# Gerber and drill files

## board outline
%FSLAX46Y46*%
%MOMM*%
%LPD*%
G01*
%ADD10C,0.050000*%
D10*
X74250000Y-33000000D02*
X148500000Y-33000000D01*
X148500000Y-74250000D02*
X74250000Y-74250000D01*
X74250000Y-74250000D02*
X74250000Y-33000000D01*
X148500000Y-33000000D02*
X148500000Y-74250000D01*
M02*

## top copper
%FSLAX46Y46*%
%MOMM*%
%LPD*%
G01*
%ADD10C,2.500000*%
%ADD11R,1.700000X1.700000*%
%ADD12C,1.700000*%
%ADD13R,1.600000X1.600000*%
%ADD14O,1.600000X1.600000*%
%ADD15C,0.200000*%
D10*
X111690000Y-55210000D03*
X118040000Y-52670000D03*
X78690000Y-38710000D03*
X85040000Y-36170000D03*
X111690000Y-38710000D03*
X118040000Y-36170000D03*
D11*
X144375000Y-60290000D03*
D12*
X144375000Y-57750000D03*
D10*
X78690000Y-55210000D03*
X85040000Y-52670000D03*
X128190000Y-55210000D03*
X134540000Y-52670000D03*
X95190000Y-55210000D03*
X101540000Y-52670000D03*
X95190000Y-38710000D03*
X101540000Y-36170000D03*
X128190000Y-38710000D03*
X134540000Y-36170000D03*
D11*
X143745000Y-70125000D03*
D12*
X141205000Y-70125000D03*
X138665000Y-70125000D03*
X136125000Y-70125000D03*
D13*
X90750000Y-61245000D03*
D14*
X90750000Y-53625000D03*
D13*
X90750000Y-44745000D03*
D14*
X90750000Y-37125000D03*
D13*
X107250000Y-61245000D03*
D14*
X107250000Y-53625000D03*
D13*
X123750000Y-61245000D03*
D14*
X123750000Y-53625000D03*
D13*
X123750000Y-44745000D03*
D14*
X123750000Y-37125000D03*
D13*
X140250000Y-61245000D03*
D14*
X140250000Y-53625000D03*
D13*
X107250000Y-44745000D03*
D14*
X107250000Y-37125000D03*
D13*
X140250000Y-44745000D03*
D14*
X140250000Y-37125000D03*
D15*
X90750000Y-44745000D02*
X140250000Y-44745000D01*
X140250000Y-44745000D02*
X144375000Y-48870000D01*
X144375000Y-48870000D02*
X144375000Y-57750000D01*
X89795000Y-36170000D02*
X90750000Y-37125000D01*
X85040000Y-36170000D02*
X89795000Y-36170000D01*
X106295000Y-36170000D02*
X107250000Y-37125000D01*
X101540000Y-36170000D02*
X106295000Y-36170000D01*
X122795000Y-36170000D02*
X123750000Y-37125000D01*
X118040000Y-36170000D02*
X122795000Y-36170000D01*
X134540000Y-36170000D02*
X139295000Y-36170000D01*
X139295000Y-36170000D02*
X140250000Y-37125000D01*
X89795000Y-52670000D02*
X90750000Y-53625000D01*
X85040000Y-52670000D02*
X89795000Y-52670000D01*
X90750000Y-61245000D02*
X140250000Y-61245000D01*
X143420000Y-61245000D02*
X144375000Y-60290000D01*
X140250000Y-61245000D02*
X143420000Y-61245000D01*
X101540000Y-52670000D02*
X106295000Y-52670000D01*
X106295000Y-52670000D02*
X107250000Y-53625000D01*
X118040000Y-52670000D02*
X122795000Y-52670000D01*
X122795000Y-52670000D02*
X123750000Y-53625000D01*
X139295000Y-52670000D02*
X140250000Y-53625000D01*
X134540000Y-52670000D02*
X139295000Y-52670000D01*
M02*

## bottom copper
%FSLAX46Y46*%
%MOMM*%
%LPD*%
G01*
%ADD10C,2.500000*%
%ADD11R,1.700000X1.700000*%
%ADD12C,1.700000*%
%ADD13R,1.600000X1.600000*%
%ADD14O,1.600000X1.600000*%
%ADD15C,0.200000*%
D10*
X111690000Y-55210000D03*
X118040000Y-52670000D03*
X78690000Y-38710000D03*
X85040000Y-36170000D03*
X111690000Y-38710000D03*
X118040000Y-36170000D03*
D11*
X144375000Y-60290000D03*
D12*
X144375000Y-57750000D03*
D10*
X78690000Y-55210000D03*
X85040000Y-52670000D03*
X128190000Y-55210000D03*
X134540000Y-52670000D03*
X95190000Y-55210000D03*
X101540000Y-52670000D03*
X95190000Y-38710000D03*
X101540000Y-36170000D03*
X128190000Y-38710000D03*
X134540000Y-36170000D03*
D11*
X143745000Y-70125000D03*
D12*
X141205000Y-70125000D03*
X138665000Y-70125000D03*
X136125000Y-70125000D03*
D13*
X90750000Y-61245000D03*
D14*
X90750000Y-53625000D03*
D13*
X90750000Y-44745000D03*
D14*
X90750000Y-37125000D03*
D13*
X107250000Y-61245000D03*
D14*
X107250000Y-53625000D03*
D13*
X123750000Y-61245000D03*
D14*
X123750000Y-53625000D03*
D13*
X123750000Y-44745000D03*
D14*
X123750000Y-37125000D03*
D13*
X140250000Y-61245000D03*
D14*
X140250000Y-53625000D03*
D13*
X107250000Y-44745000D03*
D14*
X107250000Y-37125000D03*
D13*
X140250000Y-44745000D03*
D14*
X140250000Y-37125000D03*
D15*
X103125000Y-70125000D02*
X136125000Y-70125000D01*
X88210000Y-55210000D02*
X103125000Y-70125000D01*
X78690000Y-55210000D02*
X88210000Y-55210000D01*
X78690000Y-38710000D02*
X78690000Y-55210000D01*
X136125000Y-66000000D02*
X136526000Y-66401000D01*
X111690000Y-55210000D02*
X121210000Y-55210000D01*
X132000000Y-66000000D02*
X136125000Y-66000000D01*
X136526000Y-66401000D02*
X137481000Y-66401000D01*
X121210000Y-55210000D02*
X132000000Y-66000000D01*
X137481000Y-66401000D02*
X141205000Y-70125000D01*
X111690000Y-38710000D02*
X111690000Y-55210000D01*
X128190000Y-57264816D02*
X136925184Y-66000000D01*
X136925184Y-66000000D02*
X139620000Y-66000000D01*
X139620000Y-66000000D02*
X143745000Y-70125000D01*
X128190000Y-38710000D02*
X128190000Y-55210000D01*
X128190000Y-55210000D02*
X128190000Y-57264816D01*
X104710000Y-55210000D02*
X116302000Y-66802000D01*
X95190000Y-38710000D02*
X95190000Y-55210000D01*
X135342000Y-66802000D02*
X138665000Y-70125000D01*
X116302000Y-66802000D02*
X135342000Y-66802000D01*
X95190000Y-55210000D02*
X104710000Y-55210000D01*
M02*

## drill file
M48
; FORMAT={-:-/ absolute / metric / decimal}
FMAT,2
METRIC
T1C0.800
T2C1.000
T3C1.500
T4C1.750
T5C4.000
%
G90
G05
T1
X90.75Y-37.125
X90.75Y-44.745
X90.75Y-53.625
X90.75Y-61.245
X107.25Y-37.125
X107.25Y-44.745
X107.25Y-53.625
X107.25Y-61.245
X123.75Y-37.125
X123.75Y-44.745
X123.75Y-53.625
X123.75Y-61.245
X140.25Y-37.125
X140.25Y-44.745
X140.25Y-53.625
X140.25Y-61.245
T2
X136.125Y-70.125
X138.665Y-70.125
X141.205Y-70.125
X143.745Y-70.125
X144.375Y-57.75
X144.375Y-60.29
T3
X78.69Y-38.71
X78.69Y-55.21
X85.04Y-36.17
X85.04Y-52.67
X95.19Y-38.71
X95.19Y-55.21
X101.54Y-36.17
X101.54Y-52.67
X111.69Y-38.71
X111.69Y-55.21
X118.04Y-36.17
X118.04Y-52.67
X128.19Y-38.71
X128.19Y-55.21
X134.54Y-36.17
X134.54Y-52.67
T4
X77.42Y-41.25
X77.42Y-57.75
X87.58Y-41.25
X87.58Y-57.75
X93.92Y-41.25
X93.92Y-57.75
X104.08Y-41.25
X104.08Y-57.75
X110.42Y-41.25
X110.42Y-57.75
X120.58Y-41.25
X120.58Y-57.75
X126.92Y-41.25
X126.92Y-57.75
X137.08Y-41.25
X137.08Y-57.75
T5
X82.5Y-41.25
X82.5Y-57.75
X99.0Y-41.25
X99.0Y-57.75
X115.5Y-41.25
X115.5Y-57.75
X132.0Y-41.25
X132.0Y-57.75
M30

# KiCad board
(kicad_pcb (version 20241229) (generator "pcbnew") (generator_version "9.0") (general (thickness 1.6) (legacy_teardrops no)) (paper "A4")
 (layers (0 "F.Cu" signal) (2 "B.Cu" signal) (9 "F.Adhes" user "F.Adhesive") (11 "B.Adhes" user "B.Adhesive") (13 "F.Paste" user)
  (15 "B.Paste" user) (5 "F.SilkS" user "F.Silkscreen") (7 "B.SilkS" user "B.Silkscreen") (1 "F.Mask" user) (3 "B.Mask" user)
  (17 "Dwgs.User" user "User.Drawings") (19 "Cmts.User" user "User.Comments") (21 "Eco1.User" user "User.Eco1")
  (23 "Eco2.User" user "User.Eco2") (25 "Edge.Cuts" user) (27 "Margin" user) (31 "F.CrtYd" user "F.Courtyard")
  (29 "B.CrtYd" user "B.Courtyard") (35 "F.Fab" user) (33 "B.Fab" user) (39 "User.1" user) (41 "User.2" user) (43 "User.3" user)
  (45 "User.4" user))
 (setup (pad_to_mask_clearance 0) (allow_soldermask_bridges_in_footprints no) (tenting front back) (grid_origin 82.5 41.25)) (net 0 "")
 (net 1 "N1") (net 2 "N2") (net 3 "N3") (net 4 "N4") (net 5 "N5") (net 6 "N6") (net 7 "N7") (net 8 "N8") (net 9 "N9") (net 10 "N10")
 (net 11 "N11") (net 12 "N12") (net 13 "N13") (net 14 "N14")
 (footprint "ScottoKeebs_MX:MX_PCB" (layer "F.Cu") (at 115.5 57.75)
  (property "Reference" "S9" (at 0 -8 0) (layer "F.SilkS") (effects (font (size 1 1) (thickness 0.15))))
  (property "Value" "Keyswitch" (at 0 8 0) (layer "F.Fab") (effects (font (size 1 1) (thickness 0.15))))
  (pad "" np_thru_hole circle (at -5.08 0) (size 1.75 1.75) (drill 1.75) (layers "*.Cu" "*.Mask"))
  (pad "" np_thru_hole circle (at 0 0) (size 4 4) (drill 4) (layers "*.Cu" "*.Mask"))
  (pad "" np_thru_hole circle (at 5.08 0) (size 1.75 1.75) (drill 1.75) (layers "*.Cu" "*.Mask"))
  (pad "1" thru_hole circle (at -3.81 -2.54) (size 2.5 2.5) (drill 1.5) (layers "*.Cu" "*.Mask") (remove_unused_layers no) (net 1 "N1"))
  (pad "2" thru_hole circle (at 2.54 -5.08) (size 2.5 2.5) (drill 1.5) (layers "*.Cu" "*.Mask") (remove_unused_layers no) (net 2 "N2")))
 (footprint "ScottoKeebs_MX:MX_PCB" (layer "F.Cu") (at 82.5 41.25)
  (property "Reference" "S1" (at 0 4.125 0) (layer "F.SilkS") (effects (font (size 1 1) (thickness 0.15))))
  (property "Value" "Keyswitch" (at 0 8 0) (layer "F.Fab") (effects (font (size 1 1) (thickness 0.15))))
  (pad "" np_thru_hole circle (at -5.08 0) (size 1.75 1.75) (drill 1.75) (layers "*.Cu" "*.Mask"))
  (pad "" np_thru_hole circle (at 0 0) (size 4 4) (drill 4) (layers "*.Cu" "*.Mask"))
  (pad "" np_thru_hole circle (at 5.08 0) (size 1.75 1.75) (drill 1.75) (layers "*.Cu" "*.Mask"))
  (pad "1" thru_hole circle (at -3.81 -2.54) (size 2.5 2.5) (drill 1.5) (layers "*.Cu" "*.Mask") (remove_unused_layers no) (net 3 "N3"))
  (pad "2" thru_hole circle (at 2.54 -5.08) (size 2.5 2.5) (drill 1.5) (layers "*.Cu" "*.Mask") (remove_unused_layers no) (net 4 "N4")))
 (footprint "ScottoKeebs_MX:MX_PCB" (layer "F.Cu") (at 115.5 41.25)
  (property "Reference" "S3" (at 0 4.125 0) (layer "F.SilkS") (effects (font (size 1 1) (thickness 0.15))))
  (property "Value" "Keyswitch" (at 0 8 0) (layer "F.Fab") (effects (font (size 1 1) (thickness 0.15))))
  (pad "" np_thru_hole circle (at -5.08 0) (size 1.75 1.75) (drill 1.75) (layers "*.Cu" "*.Mask"))
  (pad "" np_thru_hole circle (at 0 0) (size 4 4) (drill 4) (layers "*.Cu" "*.Mask"))
  (pad "" np_thru_hole circle (at 5.08 0) (size 1.75 1.75) (drill 1.75) (layers "*.Cu" "*.Mask"))
  (pad "1" thru_hole circle (at -3.81 -2.54) (size 2.5 2.5) (drill 1.5) (layers "*.Cu" "*.Mask") (remove_unused_layers no) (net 1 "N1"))
  (pad "2" thru_hole circle (at 2.54 -5.08) (size 2.5 2.5) (drill 1.5) (layers "*.Cu" "*.Mask") (remove_unused_layers no) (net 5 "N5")))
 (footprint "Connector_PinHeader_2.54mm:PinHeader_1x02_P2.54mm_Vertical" (layer "F.Cu") (at 144.375 60.29 180)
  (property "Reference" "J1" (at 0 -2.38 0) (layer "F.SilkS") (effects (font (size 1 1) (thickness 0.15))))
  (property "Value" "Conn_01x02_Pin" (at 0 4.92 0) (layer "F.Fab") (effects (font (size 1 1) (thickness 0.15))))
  (pad "1" thru_hole rect (at 0 0 180) (size 1.7 1.7) (drill 1) (layers "*.Cu" "*.Mask") (remove_unused_layers no) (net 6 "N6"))
  (pad "2" thru_hole circle (at 0 2.54 180) (size 1.7 1.7) (drill 1) (layers "*.Cu" "*.Mask") (remove_unused_layers no) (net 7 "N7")))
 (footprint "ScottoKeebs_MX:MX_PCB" (layer "F.Cu") (at 82.5 57.75)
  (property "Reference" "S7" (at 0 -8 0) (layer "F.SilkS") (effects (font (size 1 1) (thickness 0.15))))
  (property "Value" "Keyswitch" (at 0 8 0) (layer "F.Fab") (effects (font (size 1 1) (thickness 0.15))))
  (pad "" np_thru_hole circle (at -5.08 0) (size 1.75 1.75) (drill 1.75) (layers "*.Cu" "*.Mask"))
  (pad "" np_thru_hole circle (at 0 0) (size 4 4) (drill 4) (layers "*.Cu" "*.Mask"))
  (pad "" np_thru_hole circle (at 5.08 0) (size 1.75 1.75) (drill 1.75) (layers "*.Cu" "*.Mask"))
  (pad "1" thru_hole circle (at -3.81 -2.54) (size 2.5 2.5) (drill 1.5) (layers "*.Cu" "*.Mask") (remove_unused_layers no) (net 3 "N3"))
  (pad "2" thru_hole circle (at 2.54 -5.08) (size 2.5 2.5) (drill 1.5) (layers "*.Cu" "*.Mask") (remove_unused_layers no) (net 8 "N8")))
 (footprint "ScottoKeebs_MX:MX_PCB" (layer "F.Cu") (at 132 57.75)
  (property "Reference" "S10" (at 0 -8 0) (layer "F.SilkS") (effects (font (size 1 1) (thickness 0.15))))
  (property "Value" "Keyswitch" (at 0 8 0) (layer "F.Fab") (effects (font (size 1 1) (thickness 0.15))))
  (pad "" np_thru_hole circle (at -5.08 0) (size 1.75 1.75) (drill 1.75) (layers "*.Cu" "*.Mask"))
  (pad "" np_thru_hole circle (at 0 0) (size 4 4) (drill 4) (layers "*.Cu" "*.Mask"))
  (pad "" np_thru_hole circle (at 5.08 0) (size 1.75 1.75) (drill 1.75) (layers "*.Cu" "*.Mask"))
  (pad "1" thru_hole circle (at -3.81 -2.54) (size 2.5 2.5) (drill 1.5) (layers "*.Cu" "*.Mask") (remove_unused_layers no) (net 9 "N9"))
  (pad "2" thru_hole circle (at 2.54 -5.08) (size 2.5 2.5) (drill 1.5) (layers "*.Cu" "*.Mask") (remove_unused_layers no) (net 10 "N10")))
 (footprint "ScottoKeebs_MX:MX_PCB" (layer "F.Cu") (at 99 57.75)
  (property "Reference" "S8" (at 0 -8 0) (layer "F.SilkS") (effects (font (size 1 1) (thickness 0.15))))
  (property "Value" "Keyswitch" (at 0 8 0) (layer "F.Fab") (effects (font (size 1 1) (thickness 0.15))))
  (pad "" np_thru_hole circle (at -5.08 0) (size 1.75 1.75) (drill 1.75) (layers "*.Cu" "*.Mask"))
  (pad "" np_thru_hole circle (at 0 0) (size 4 4) (drill 4) (layers "*.Cu" "*.Mask"))
  (pad "" np_thru_hole circle (at 5.08 0) (size 1.75 1.75) (drill 1.75) (layers "*.Cu" "*.Mask"))
  (pad "1" thru_hole circle (at -3.81 -2.54) (size 2.5 2.5) (drill 1.5) (layers "*.Cu" "*.Mask") (remove_unused_layers no) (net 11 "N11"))
  (pad "2" thru_hole circle (at 2.54 -5.08) (size 2.5 2.5) (drill 1.5) (layers "*.Cu" "*.Mask") (remove_unused_layers no) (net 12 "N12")))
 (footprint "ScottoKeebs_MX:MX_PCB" (layer "F.Cu") (at 99 41.25)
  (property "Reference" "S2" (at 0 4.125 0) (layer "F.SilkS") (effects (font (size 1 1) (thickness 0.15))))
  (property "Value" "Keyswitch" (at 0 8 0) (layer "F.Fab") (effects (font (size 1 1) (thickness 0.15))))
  (pad "" np_thru_hole circle (at -5.08 0) (size 1.75 1.75) (drill 1.75) (layers "*.Cu" "*.Mask"))
  (pad "" np_thru_hole circle (at 0 0) (size 4 4) (drill 4) (layers "*.Cu" "*.Mask"))
  (pad "" np_thru_hole circle (at 5.08 0) (size 1.75 1.75) (drill 1.75) (layers "*.Cu" "*.Mask"))
  (pad "1" thru_hole circle (at -3.81 -2.54) (size 2.5 2.5) (drill 1.5) (layers "*.Cu" "*.Mask") (remove_unused_layers no) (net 11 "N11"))
  (pad "2" thru_hole circle (at 2.54 -5.08) (size 2.5 2.5) (drill 1.5) (layers "*.Cu" "*.Mask") (remove_unused_layers no) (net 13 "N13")))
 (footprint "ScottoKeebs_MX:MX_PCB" (layer "F.Cu") (at 132 41.25)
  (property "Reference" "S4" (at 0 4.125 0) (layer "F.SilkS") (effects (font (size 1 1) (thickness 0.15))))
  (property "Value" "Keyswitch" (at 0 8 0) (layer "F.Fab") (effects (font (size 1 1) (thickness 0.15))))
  (pad "" np_thru_hole circle (at -5.08 0) (size 1.75 1.75) (drill 1.75) (layers "*.Cu" "*.Mask"))
  (pad "" np_thru_hole circle (at 0 0) (size 4 4) (drill 4) (layers "*.Cu" "*.Mask"))
  (pad "" np_thru_hole circle (at 5.08 0) (size 1.75 1.75) (drill 1.75) (layers "*.Cu" "*.Mask"))
  (pad "1" thru_hole circle (at -3.81 -2.54) (size 2.5 2.5) (drill 1.5) (layers "*.Cu" "*.Mask") (remove_unused_layers no) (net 9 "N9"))
  (pad "2" thru_hole circle (at 2.54 -5.08) (size 2.5 2.5) (drill 1.5) (layers "*.Cu" "*.Mask") (remove_unused_layers no) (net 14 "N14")))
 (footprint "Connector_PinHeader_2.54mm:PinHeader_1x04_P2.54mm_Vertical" (layer "F.Cu") (at 143.745 70.125 -90)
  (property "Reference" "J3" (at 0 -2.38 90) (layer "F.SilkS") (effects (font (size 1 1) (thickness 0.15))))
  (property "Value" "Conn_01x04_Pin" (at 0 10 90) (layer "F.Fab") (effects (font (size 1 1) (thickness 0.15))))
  (pad "1" thru_hole rect (at 0 0 270) (size 1.7 1.7) (drill 1) (layers "*.Cu" "*.Mask") (remove_unused_layers no) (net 9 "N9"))
  (pad "2" thru_hole circle (at 0 2.54 270) (size 1.7 1.7) (drill 1) (layers "*.Cu" "*.Mask") (remove_unused_layers no) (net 1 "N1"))
  (pad "3" thru_hole circle (at 0 5.08 270) (size 1.7 1.7) (drill 1) (layers "*.Cu" "*.Mask") (remove_unused_layers no) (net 11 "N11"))
  (pad "4" thru_hole circle (at 0 7.62 270) (size 1.7 1.7) (drill 1) (layers "*.Cu" "*.Mask") (remove_unused_layers no) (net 3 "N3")))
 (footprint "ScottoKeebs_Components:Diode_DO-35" (layer "B.Cu") (at 90.75 61.245 90)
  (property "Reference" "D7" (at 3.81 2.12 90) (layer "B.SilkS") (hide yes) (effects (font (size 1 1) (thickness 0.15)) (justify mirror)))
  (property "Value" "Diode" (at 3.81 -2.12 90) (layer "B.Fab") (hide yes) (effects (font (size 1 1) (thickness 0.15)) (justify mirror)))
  (pad "1" thru_hole rect (at 0 0 90) (size 1.6 1.6) (drill 0.8) (layers "*.Cu" "*.Mask") (remove_unused_layers no) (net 6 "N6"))
  (pad "2" thru_hole oval (at 7.62 0 90) (size 1.6 1.6) (drill 0.8) (layers "*.Cu" "*.Mask") (remove_unused_layers no) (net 8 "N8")))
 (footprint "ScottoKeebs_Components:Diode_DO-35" (layer "B.Cu") (at 90.75 44.745 90)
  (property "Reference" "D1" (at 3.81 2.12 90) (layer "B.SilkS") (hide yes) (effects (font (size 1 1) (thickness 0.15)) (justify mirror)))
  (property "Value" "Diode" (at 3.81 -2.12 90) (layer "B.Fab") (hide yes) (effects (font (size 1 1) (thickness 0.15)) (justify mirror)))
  (pad "1" thru_hole rect (at 0 0 90) (size 1.6 1.6) (drill 0.8) (layers "*.Cu" "*.Mask") (remove_unused_layers no) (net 7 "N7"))
  (pad "2" thru_hole oval (at 7.62 0 90) (size 1.6 1.6) (drill 0.8) (layers "*.Cu" "*.Mask") (remove_unused_layers no) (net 4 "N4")))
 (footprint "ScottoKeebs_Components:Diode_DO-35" (layer "B.Cu") (at 107.25 61.245 90)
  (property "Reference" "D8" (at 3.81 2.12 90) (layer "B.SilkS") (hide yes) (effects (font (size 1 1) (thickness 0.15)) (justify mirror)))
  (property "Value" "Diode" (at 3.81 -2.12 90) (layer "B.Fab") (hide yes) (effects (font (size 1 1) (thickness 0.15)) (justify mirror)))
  (pad "1" thru_hole rect (at 0 0 90) (size 1.6 1.6) (drill 0.8) (layers "*.Cu" "*.Mask") (remove_unused_layers no) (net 6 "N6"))
  (pad "2" thru_hole oval (at 7.62 0 90) (size 1.6 1.6) (drill 0.8) (layers "*.Cu" "*.Mask") (remove_unused_layers no) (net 12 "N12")))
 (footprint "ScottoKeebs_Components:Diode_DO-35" (layer "B.Cu") (at 123.75 61.245 90)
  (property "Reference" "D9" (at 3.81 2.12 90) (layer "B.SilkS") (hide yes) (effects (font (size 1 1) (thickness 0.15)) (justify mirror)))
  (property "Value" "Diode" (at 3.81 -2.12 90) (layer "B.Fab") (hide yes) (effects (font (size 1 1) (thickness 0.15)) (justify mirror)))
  (pad "1" thru_hole rect (at 0 0 90) (size 1.6 1.6) (drill 0.8) (layers "*.Cu" "*.Mask") (remove_unused_layers no) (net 6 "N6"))
  (pad "2" thru_hole oval (at 7.62 0 90) (size 1.6 1.6) (drill 0.8) (layers "*.Cu" "*.Mask") (remove_unused_layers no) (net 2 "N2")))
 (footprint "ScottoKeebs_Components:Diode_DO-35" (layer "B.Cu") (at 123.75 44.745 90)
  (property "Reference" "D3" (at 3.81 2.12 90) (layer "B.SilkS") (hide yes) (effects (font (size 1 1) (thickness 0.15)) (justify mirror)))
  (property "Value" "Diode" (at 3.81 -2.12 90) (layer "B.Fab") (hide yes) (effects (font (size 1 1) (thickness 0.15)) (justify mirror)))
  (pad "1" thru_hole rect (at 0 0 90) (size 1.6 1.6) (drill 0.8) (layers "*.Cu" "*.Mask") (remove_unused_layers no) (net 7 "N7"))
  (pad "2" thru_hole oval (at 7.62 0 90) (size 1.6 1.6) (drill 0.8) (layers "*.Cu" "*.Mask") (remove_unused_layers no) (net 5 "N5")))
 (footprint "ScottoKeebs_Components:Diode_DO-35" (layer "B.Cu") (at 140.25 61.245 90)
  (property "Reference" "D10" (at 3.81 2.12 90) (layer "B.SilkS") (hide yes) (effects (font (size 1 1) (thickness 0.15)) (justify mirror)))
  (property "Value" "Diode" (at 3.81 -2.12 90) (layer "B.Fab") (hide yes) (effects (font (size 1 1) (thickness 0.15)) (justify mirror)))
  (pad "1" thru_hole rect (at 0 0 90) (size 1.6 1.6) (drill 0.8) (layers "*.Cu" "*.Mask") (remove_unused_layers no) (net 6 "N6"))
  (pad "2" thru_hole oval (at 7.62 0 90) (size 1.6 1.6) (drill 0.8) (layers "*.Cu" "*.Mask") (remove_unused_layers no) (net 10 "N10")))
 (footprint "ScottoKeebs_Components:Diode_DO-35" (layer "B.Cu") (at 107.25 44.745 90)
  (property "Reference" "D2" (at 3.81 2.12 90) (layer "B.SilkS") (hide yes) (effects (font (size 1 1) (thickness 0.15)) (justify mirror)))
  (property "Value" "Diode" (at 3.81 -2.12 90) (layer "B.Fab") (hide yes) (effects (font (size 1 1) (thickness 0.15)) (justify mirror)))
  (pad "1" thru_hole rect (at 0 0 90) (size 1.6 1.6) (drill 0.8) (layers "*.Cu" "*.Mask") (remove_unused_layers no) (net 7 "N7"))
  (pad "2" thru_hole oval (at 7.62 0 90) (size 1.6 1.6) (drill 0.8) (layers "*.Cu" "*.Mask") (remove_unused_layers no) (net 13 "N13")))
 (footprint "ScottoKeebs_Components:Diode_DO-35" (layer "B.Cu") (at 140.25 44.745 90)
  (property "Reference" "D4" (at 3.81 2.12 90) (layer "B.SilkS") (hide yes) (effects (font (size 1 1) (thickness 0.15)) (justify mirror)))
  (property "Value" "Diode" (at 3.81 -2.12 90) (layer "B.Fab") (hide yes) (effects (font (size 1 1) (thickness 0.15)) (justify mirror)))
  (pad "1" thru_hole rect (at 0 0 90) (size 1.6 1.6) (drill 0.8) (layers "*.Cu" "*.Mask") (remove_unused_layers no) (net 7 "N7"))
  (pad "2" thru_hole oval (at 7.62 0 90) (size 1.6 1.6) (drill 0.8) (layers "*.Cu" "*.Mask") (remove_unused_layers no) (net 14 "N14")))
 (gr_line (start 74.25 33) (end 148.5 33) (stroke (width 0.05) (type default)) (layer "Edge.Cuts"))
 (gr_line (start 148.5 74.25) (end 74.25 74.25) (stroke (width 0.05) (type default)) (layer "Edge.Cuts"))
 (gr_line (start 74.25 74.25) (end 74.25 33) (stroke (width 0.05) (type default)) (layer "Edge.Cuts"))
 (gr_line (start 148.5 33) (end 148.5 74.25) (stroke (width 0.05) (type default)) (layer "Edge.Cuts"))
 (segment (start 90.75 44.745) (end 140.25 44.745) (width 0.2) (layer "F.Cu") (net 7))
 (segment (start 140.25 44.745) (end 144.375 48.87) (width 0.2) (layer "F.Cu") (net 7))
 (segment (start 144.375 48.87) (end 144.375 57.75) (width 0.2) (layer "F.Cu") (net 7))
 (segment (start 89.795 36.17) (end 90.75 37.125) (width 0.2) (layer "F.Cu") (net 4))
 (segment (start 85.04 36.17) (end 89.795 36.17) (width 0.2) (layer "F.Cu") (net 4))
 (segment (start 106.295 36.17) (end 107.25 37.125) (width 0.2) (layer "F.Cu") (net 13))
 (segment (start 101.54 36.17) (end 106.295 36.17) (width 0.2) (layer "F.Cu") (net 13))
 (segment (start 122.795 36.17) (end 123.75 37.125) (width 0.2) (layer "F.Cu") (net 5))
 (segment (start 118.04 36.17) (end 122.795 36.17) (width 0.2) (layer "F.Cu") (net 5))
 (segment (start 134.54 36.17) (end 139.295 36.17) (width 0.2) (layer "F.Cu") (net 14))
 (segment (start 139.295 36.17) (end 140.25 37.125) (width 0.2) (layer "F.Cu") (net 14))
 (segment (start 89.795 52.67) (end 90.75 53.625) (width 0.2) (layer "F.Cu") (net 8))
 (segment (start 85.04 52.67) (end 89.795 52.67) (width 0.2) (layer "F.Cu") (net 8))
 (segment (start 90.75 61.245) (end 140.25 61.245) (width 0.2) (layer "F.Cu") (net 6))
 (segment (start 143.42 61.245) (end 144.375 60.29) (width 0.2) (layer "F.Cu") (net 6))
 (segment (start 140.25 61.245) (end 143.42 61.245) (width 0.2) (layer "F.Cu") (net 6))
 (segment (start 101.54 52.67) (end 106.295 52.67) (width 0.2) (layer "F.Cu") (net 12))
 (segment (start 106.295 52.67) (end 107.25 53.625) (width 0.2) (layer "F.Cu") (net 12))
 (segment (start 118.04 52.67) (end 122.795 52.67) (width 0.2) (layer "F.Cu") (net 2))
 (segment (start 122.795 52.67) (end 123.75 53.625) (width 0.2) (layer "F.Cu") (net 2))
 (segment (start 139.295 52.67) (end 140.25 53.625) (width 0.2) (layer "F.Cu") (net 10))
 (segment (start 134.54 52.67) (end 139.295 52.67) (width 0.2) (layer "F.Cu") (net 10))
 (segment (start 103.125 70.125) (end 136.125 70.125) (width 0.2) (layer "B.Cu") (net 3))
 (segment (start 88.21 55.21) (end 103.125 70.125) (width 0.2) (layer "B.Cu") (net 3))
 (segment (start 78.69 55.21) (end 88.21 55.21) (width 0.2) (layer "B.Cu") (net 3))
 (segment (start 78.69 38.71) (end 78.69 55.21) (width 0.2) (layer "B.Cu") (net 3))
 (segment (start 136.125 66) (end 136.526 66.401) (width 0.2) (layer "B.Cu") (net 1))
 (segment (start 111.69 55.21) (end 121.21 55.21) (width 0.2) (layer "B.Cu") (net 1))
 (segment (start 132 66) (end 136.125 66) (width 0.2) (layer "B.Cu") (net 1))
 (segment (start 136.526 66.401) (end 137.481 66.401) (width 0.2) (layer "B.Cu") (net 1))
 (segment (start 121.21 55.21) (end 132 66) (width 0.2) (layer "B.Cu") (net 1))
 (segment (start 137.481 66.401) (end 141.205 70.125) (width 0.2) (layer "B.Cu") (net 1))
 (segment (start 111.69 38.71) (end 111.69 55.21) (width 0.2) (layer "B.Cu") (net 1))
 (segment (start 128.19 57.264816) (end 136.925184 66) (width 0.2) (layer "B.Cu") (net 9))
 (segment (start 136.925184 66) (end 139.62 66) (width 0.2) (layer "B.Cu") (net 9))
 (segment (start 139.62 66) (end 143.745 70.125) (width 0.2) (layer "B.Cu") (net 9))
 (segment (start 128.19 38.71) (end 128.19 55.21) (width 0.2) (layer "B.Cu") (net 9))
 (segment (start 128.19 55.21) (end 128.19 57.264816) (width 0.2) (layer "B.Cu") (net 9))
 (segment (start 104.71 55.21) (end 116.302 66.802) (width 0.2) (layer "B.Cu") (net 11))
 (segment (start 95.19 38.71) (end 95.19 55.21) (width 0.2) (layer "B.Cu") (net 11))
 (segment (start 135.342 66.802) (end 138.665 70.125) (width 0.2) (layer "B.Cu") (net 11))
 (segment (start 116.302 66.802) (end 135.342 66.802) (width 0.2) (layer "B.Cu") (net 11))
 (segment (start 95.19 55.21) (end 104.71 55.21) (width 0.2) (layer "B.Cu") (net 11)))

